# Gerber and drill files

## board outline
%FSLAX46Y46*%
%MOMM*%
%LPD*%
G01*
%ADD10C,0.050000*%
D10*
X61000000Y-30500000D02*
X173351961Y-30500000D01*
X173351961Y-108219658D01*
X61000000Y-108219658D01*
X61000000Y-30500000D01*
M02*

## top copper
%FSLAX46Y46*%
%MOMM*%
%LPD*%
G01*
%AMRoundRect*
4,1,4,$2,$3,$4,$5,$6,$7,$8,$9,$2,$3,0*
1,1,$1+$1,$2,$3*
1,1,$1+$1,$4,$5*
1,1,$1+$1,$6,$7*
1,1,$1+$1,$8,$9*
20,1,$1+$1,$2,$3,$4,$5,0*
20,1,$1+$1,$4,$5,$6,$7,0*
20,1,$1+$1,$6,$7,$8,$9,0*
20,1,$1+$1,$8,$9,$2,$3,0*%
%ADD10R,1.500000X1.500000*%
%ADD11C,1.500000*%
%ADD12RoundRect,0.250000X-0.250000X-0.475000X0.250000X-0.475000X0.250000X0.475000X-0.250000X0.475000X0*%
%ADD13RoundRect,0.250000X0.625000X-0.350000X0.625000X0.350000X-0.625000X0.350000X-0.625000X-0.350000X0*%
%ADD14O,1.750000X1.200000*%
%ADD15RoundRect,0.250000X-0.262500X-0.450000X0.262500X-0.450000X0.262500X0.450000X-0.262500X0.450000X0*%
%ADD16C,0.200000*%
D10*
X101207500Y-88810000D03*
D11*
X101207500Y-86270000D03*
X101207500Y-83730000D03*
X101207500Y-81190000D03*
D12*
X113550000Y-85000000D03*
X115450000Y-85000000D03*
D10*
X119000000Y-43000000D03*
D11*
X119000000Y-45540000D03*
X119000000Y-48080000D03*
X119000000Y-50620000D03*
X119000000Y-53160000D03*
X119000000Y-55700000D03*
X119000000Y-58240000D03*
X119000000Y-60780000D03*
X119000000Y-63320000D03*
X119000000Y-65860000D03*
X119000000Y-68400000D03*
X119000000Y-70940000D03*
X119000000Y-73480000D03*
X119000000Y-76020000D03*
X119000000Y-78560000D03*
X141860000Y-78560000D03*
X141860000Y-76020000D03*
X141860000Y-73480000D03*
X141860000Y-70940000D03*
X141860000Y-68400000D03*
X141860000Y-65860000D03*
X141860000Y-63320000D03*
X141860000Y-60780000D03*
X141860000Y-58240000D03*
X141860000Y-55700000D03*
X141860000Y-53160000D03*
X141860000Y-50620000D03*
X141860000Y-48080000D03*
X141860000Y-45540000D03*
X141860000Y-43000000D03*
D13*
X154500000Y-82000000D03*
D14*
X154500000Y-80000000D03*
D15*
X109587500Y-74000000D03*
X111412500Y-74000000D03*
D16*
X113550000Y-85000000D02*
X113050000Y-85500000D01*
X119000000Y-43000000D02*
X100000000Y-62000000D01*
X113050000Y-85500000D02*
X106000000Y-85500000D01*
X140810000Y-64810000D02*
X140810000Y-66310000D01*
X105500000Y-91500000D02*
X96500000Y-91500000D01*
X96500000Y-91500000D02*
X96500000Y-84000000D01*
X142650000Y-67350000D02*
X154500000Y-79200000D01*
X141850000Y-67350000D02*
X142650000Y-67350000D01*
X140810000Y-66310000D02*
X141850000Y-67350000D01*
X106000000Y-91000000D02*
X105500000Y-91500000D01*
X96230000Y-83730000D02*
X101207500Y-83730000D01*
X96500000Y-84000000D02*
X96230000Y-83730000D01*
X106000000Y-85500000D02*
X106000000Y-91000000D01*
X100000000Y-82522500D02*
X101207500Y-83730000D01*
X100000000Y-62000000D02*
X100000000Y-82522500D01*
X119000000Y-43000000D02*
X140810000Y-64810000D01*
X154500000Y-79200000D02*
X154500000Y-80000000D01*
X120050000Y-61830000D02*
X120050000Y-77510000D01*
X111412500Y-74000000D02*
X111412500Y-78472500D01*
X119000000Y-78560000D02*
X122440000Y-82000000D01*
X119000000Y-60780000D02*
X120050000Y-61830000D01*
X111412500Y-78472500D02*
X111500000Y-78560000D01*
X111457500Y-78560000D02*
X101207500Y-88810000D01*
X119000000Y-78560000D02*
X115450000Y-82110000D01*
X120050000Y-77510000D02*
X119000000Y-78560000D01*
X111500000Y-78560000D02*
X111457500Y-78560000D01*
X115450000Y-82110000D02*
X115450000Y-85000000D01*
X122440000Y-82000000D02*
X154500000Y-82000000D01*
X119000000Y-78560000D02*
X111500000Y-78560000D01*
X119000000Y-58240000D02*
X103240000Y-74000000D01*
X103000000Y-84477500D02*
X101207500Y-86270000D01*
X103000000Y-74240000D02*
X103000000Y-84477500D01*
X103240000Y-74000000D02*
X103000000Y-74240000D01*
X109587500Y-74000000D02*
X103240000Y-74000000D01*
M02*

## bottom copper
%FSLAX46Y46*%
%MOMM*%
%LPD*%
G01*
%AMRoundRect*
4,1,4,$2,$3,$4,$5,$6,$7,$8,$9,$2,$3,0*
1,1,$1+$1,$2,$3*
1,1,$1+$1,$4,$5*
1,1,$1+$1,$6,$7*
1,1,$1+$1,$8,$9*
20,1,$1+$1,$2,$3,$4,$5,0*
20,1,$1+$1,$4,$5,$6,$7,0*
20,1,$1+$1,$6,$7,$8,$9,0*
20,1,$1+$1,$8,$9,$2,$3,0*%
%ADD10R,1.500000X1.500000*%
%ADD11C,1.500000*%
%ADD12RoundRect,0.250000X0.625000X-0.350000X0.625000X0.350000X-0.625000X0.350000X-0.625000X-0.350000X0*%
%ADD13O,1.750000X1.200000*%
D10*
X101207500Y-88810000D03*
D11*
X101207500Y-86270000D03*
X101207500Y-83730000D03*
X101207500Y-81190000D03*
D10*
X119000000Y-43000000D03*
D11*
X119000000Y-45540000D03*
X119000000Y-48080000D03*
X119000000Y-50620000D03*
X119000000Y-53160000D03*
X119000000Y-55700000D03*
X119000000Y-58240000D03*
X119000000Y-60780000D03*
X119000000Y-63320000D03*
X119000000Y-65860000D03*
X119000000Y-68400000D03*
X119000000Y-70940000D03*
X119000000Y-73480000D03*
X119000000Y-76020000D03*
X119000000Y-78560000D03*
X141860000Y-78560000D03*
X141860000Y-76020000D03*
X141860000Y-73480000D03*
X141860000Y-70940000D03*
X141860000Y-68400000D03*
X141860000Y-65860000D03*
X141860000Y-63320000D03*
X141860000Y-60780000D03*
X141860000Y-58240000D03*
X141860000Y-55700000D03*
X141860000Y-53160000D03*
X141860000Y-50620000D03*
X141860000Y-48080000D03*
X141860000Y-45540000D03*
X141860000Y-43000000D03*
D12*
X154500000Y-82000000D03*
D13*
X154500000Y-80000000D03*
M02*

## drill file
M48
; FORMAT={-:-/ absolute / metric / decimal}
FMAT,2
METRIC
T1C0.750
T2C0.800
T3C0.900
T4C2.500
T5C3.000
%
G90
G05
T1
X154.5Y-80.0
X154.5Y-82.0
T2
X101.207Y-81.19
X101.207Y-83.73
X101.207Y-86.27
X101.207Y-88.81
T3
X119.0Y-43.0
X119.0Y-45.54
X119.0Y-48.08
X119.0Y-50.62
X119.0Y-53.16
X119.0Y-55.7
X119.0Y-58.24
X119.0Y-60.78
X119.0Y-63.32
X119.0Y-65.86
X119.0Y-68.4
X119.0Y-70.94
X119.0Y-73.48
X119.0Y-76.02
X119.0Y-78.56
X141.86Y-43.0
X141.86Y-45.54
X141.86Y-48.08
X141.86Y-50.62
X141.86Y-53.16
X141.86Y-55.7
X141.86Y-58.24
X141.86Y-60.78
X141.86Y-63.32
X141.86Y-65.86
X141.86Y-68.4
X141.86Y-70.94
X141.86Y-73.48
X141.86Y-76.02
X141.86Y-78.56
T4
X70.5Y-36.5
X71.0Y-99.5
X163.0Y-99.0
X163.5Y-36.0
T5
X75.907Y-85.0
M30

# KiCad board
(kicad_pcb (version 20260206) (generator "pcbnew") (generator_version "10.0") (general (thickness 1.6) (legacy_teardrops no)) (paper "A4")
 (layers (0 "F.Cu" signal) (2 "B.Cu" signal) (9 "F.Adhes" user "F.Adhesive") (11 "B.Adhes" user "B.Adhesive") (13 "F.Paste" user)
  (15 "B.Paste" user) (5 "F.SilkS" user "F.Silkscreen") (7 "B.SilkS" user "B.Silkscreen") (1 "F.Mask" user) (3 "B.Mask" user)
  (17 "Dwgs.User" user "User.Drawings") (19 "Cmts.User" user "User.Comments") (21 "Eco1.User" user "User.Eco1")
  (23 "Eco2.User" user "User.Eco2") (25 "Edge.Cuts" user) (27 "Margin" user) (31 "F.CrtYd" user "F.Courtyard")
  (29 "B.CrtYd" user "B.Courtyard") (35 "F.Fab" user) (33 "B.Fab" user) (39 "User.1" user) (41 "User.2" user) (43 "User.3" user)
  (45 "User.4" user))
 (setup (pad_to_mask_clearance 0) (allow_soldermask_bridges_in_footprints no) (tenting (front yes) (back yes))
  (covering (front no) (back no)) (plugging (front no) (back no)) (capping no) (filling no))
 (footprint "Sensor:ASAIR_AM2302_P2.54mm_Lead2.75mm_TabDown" (layer "F.Cu") (at 101.2075 88.81 180)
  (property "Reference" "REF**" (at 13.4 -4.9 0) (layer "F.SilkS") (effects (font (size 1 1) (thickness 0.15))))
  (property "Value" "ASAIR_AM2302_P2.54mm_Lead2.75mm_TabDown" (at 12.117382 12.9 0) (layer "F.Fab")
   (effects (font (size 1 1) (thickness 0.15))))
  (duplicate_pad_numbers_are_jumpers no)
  (pad "" np_thru_hole circle (at 25.3 3.81 180) (size 3 3) (drill 3) (layers "*.Cu" "*.Mask"))
  (pad "1" thru_hole rect (at 0 0 180) (size 1.5 1.5) (drill 0.8) (layers "*.Cu" "*.Mask") (remove_unused_layers no) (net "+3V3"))
  (pad "2" thru_hole circle (at 0 2.54 180) (size 1.5 1.5) (drill 0.8) (layers "*.Cu" "*.Mask") (remove_unused_layers no) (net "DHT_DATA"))
  (pad "3" thru_hole circle (at 0 5.08 180) (size 1.5 1.5) (drill 0.8) (layers "*.Cu" "*.Mask") (remove_unused_layers no) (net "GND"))
  (pad "4" thru_hole circle (at 0 7.62 180) (size 1.5 1.5) (drill 0.8) (layers "*.Cu" "*.Mask") (remove_unused_layers no)))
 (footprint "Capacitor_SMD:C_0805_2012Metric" (layer "F.Cu") (at 114.5 85)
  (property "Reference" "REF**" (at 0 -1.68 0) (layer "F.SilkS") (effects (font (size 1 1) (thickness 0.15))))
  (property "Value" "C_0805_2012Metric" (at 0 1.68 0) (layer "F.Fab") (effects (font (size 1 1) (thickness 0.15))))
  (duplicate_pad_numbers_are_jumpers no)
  (pad "1" smd roundrect (at -0.95 0) (size 1 1.45) (layers "F.Cu" "F.Mask" "F.Paste") (roundrect_rratio 0.25) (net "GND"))
  (pad "2" smd roundrect (at 0.95 0) (size 1 1.45) (layers "F.Cu" "F.Mask" "F.Paste") (roundrect_rratio 0.25) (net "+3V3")))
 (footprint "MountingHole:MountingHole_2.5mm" (layer "F.Cu") (at 163 99)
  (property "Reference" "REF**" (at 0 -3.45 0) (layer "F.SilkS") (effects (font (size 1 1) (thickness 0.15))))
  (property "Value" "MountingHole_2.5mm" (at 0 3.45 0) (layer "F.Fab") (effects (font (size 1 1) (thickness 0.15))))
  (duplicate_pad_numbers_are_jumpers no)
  (pad "" np_thru_hole circle (at 0 0) (size 2.5 2.5) (drill 2.5) (layers "*.Cu" "*.Mask")))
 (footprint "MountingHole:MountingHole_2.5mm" (layer "F.Cu") (at 71 99.5)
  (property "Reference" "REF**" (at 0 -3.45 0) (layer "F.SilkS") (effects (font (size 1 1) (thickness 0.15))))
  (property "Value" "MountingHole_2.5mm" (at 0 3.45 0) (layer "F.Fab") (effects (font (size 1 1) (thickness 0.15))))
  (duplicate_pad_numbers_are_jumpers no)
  (pad "" np_thru_hole circle (at 0 0) (size 2.5 2.5) (drill 2.5) (layers "*.Cu" "*.Mask")))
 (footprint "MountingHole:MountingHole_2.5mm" (layer "F.Cu") (at 163.5 36)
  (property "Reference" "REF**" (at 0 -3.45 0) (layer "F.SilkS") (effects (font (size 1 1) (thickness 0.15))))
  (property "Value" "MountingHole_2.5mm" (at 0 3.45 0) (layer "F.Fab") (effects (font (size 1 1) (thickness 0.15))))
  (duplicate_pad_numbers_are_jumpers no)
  (pad "" np_thru_hole circle (at 0 0) (size 2.5 2.5) (drill 2.5) (layers "*.Cu" "*.Mask")))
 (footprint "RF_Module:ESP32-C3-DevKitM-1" (layer "F.Cu") (at 119 43)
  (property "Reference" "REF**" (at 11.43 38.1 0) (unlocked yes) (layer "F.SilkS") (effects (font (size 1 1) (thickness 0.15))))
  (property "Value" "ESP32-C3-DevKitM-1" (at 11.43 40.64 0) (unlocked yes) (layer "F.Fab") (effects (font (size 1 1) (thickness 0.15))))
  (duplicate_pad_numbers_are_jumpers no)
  (pad "1" thru_hole rect (at 0 0) (size 1.5 1.5) (drill 0.9) (layers "*.Cu" "*.Mask") (remove_unused_layers yes) (keep_end_layers yes)
   (zone_layer_connections) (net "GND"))
  (pad "2" thru_hole circle (at 0 2.54) (size 1.5 1.5) (drill 0.9) (layers "*.Cu" "*.Mask") (remove_unused_layers yes) (keep_end_layers yes)
   (zone_layer_connections))
  (pad "3" thru_hole circle (at 0 5.08) (size 1.5 1.5) (drill 0.9) (layers "*.Cu" "*.Mask") (remove_unused_layers yes) (keep_end_layers yes)
   (zone_layer_connections))
  (pad "4" thru_hole circle (at 0 7.62) (size 1.5 1.5) (drill 0.9) (layers "*.Cu" "*.Mask") (remove_unused_layers yes) (keep_end_layers yes)
   (zone_layer_connections))
  (pad "5" thru_hole circle (at 0 10.16) (size 1.5 1.5) (drill 0.9) (layers "*.Cu" "*.Mask") (remove_unused_layers yes)
   (keep_end_layers yes) (zone_layer_connections))
  (pad "6" thru_hole circle (at 0 12.7) (size 1.5 1.5) (drill 0.9) (layers "*.Cu" "*.Mask") (remove_unused_layers yes) (keep_end_layers yes)
   (zone_layer_connections))
  (pad "7" thru_hole circle (at 0 15.24) (size 1.5 1.5) (drill 0.9) (layers "*.Cu" "*.Mask") (remove_unused_layers yes)
   (keep_end_layers yes) (zone_layer_connections) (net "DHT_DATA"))
  (pad "8" thru_hole circle (at 0 17.78) (size 1.5 1.5) (drill 0.9) (layers "*.Cu" "*.Mask") (remove_unused_layers yes)
   (keep_end_layers yes) (zone_layer_connections) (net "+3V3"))
  (pad "9" thru_hole circle (at 0 20.32) (size 1.5 1.5) (drill 0.9) (layers "*.Cu" "*.Mask") (remove_unused_layers yes)
   (keep_end_layers yes) (zone_layer_connections))
  (pad "10" thru_hole circle (at 0 22.86) (size 1.5 1.5) (drill 0.9) (layers "*.Cu" "*.Mask") (remove_unused_layers yes)
   (keep_end_layers yes) (zone_layer_connections))
  (pad "11" thru_hole circle (at 0 25.4) (size 1.5 1.5) (drill 0.9) (layers "*.Cu" "*.Mask") (remove_unused_layers yes)
   (keep_end_layers yes) (zone_layer_connections))
  (pad "12" thru_hole circle (at 0 27.94) (size 1.5 1.5) (drill 0.9) (layers "*.Cu" "*.Mask") (remove_unused_layers yes)
   (keep_end_layers yes) (zone_layer_connections))
  (pad "13" thru_hole circle (at 0 30.48) (size 1.5 1.5) (drill 0.9) (layers "*.Cu" "*.Mask") (remove_unused_layers yes)
   (keep_end_layers yes) (zone_layer_connections))
  (pad "14" thru_hole circle (at 0 33.02) (size 1.5 1.5) (drill 0.9) (layers "*.Cu" "*.Mask") (remove_unused_layers yes)
   (keep_end_layers yes) (zone_layer_connections))
  (pad "15" thru_hole circle (at 0 35.56) (size 1.5 1.5) (drill 0.9) (layers "*.Cu" "*.Mask") (remove_unused_layers yes)
   (keep_end_layers yes) (zone_layer_connections) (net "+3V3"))
  (pad "16" thru_hole circle (at 22.86 35.56) (size 1.5 1.5) (drill 0.9) (layers "*.Cu" "*.Mask") (remove_unused_layers yes)
   (keep_end_layers yes) (zone_layer_connections))
  (pad "17" thru_hole circle (at 22.86 33.02) (size 1.5 1.5) (drill 0.9) (layers "*.Cu" "*.Mask") (remove_unused_layers yes)
   (keep_end_layers yes) (zone_layer_connections))
  (pad "18" thru_hole circle (at 22.86 30.48) (size 1.5 1.5) (drill 0.9) (layers "*.Cu" "*.Mask") (remove_unused_layers yes)
   (keep_end_layers yes) (zone_layer_connections))
  (pad "19" thru_hole circle (at 22.86 27.94) (size 1.5 1.5) (drill 0.9) (layers "*.Cu" "*.Mask") (remove_unused_layers yes)
   (keep_end_layers yes) (zone_layer_connections))
  (pad "20" thru_hole circle (at 22.86 25.4) (size 1.5 1.5) (drill 0.9) (layers "*.Cu" "*.Mask") (remove_unused_layers yes)
   (keep_end_layers yes) (zone_layer_connections))
  (pad "21" thru_hole circle (at 22.86 22.86) (size 1.5 1.5) (drill 0.9) (layers "*.Cu" "*.Mask") (remove_unused_layers yes)
   (keep_end_layers yes) (zone_layer_connections))
  (pad "22" thru_hole circle (at 22.86 20.32) (size 1.5 1.5) (drill 0.9) (layers "*.Cu" "*.Mask") (remove_unused_layers yes)
   (keep_end_layers yes) (zone_layer_connections))
  (pad "23" thru_hole circle (at 22.86 17.78) (size 1.5 1.5) (drill 0.9) (layers "*.Cu" "*.Mask") (remove_unused_layers yes)
   (keep_end_layers yes) (zone_layer_connections))
  (pad "24" thru_hole circle (at 22.86 15.24) (size 1.5 1.5) (drill 0.9) (layers "*.Cu" "*.Mask") (remove_unused_layers yes)
   (keep_end_layers yes) (zone_layer_connections))
  (pad "25" thru_hole circle (at 22.86 12.7) (size 1.5 1.5) (drill 0.9) (layers "*.Cu" "*.Mask") (remove_unused_layers yes)
   (keep_end_layers yes) (zone_layer_connections))
  (pad "26" thru_hole circle (at 22.86 10.16) (size 1.5 1.5) (drill 0.9) (layers "*.Cu" "*.Mask") (remove_unused_layers yes)
   (keep_end_layers yes) (zone_layer_connections))
  (pad "27" thru_hole circle (at 22.86 7.62) (size 1.5 1.5) (drill 0.9) (layers "*.Cu" "*.Mask") (remove_unused_layers yes)
   (keep_end_layers yes) (zone_layer_connections))
  (pad "28" thru_hole circle (at 22.86 5.08) (size 1.5 1.5) (drill 0.9) (layers "*.Cu" "*.Mask") (remove_unused_layers yes)
   (keep_end_layers yes) (zone_layer_connections))
  (pad "29" thru_hole circle (at 22.86 2.54) (size 1.5 1.5) (drill 0.9) (layers "*.Cu" "*.Mask") (remove_unused_layers yes)
   (keep_end_layers yes) (zone_layer_connections))
  (pad "30" thru_hole circle (at 22.86 0) (size 1.5 1.5) (drill 0.9) (layers "*.Cu" "*.Mask") (remove_unused_layers yes)
   (keep_end_layers yes) (zone_layer_connections)))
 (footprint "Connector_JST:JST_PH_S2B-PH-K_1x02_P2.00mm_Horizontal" (layer "F.Cu") (at 154.5 82 90)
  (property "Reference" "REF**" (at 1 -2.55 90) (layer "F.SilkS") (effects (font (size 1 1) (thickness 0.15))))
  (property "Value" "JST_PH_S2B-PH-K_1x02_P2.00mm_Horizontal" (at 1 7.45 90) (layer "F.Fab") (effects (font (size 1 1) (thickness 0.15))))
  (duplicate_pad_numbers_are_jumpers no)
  (pad "1" thru_hole roundrect (at 0 0 90) (size 1.2 1.75) (drill 0.75) (layers "*.Cu" "*.Mask") (remove_unused_layers no)
   (roundrect_rratio 0.208333) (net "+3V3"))
  (pad "2" thru_hole oval (at 2 0 90) (size 1.2 1.75) (drill 0.75) (layers "*.Cu" "*.Mask") (remove_unused_layers no) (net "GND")))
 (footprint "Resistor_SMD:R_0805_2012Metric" (layer "F.Cu") (at 110.5 74)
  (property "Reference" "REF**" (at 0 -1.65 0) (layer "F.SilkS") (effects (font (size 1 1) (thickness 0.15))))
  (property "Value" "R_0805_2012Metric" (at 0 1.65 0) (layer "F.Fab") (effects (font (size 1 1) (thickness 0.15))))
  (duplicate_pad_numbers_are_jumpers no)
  (pad "1" smd roundrect (at -0.9125 0) (size 1.025 1.4) (layers "F.Cu" "F.Mask" "F.Paste") (roundrect_rratio 0.243902) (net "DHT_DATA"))
  (pad "2" smd roundrect (at 0.9125 0) (size 1.025 1.4) (layers "F.Cu" "F.Mask" "F.Paste") (roundrect_rratio 0.243902) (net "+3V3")))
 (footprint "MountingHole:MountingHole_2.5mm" (layer "F.Cu") (at 70.5 36.5)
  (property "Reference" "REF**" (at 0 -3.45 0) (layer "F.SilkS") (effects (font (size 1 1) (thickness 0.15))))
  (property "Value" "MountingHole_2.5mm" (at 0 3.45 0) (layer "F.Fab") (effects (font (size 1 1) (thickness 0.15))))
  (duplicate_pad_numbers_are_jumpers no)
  (pad "" np_thru_hole circle (at 0 0) (size 2.5 2.5) (drill 2.5) (layers "*.Cu" "*.Mask")))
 (gr_rect (start 61 30.5) (end 173.351961 108.219658) (stroke (width 0.05) (type default)) (fill no) (layer "Edge.Cuts"))
 (segment (start 113.55 85) (end 113.05 85.5) (width 0.2) (layer "F.Cu") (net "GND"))
 (segment (start 119 43) (end 100 62) (width 0.2) (layer "F.Cu") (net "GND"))
 (segment (start 113.05 85.5) (end 106 85.5) (width 0.2) (layer "F.Cu") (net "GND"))
 (segment (start 140.81 64.81) (end 140.81 66.31) (width 0.2) (layer "F.Cu") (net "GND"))
 (segment (start 105.5 91.5) (end 96.5 91.5) (width 0.2) (layer "F.Cu") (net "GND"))
 (segment (start 96.5 91.5) (end 96.5 84) (width 0.2) (layer "F.Cu") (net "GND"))
 (segment (start 142.65 67.35) (end 154.5 79.2) (width 0.2) (layer "F.Cu") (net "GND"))
 (segment (start 141.85 67.35) (end 142.65 67.35) (width 0.2) (layer "F.Cu") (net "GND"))
 (segment (start 140.81 66.31) (end 141.85 67.35) (width 0.2) (layer "F.Cu") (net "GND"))
 (segment (start 106 91) (end 105.5 91.5) (width 0.2) (layer "F.Cu") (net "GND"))
 (segment (start 96.23 83.73) (end 101.2075 83.73) (width 0.2) (layer "F.Cu") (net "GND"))
 (segment (start 96.5 84) (end 96.23 83.73) (width 0.2) (layer "F.Cu") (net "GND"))
 (segment (start 106 85.5) (end 106 91) (width 0.2) (layer "F.Cu") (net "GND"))
 (segment (start 100 82.5225) (end 101.2075 83.73) (width 0.2) (layer "F.Cu") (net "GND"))
 (segment (start 100 62) (end 100 82.5225) (width 0.2) (layer "F.Cu") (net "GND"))
 (segment (start 119 43) (end 140.81 64.81) (width 0.2) (layer "F.Cu") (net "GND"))
 (segment (start 154.5 79.2) (end 154.5 80) (width 0.2) (layer "F.Cu") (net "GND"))
 (segment (start 120.05 61.83) (end 120.05 77.51) (width 0.2) (layer "F.Cu") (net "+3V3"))
 (segment (start 111.4125 74) (end 111.4125 78.4725) (width 0.2) (layer "F.Cu") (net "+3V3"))
 (segment (start 119 78.56) (end 122.44 82) (width 0.2) (layer "F.Cu") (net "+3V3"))
 (segment (start 119 60.78) (end 120.05 61.83) (width 0.2) (layer "F.Cu") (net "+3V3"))
 (segment (start 111.4125 78.4725) (end 111.5 78.56) (width 0.2) (layer "F.Cu") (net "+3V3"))
 (segment (start 111.4575 78.56) (end 101.2075 88.81) (width 0.2) (layer "F.Cu") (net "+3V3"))
 (segment (start 119 78.56) (end 115.45 82.11) (width 0.2) (layer "F.Cu") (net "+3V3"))
 (segment (start 120.05 77.51) (end 119 78.56) (width 0.2) (layer "F.Cu") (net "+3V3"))
 (segment (start 111.5 78.56) (end 111.4575 78.56) (width 0.2) (layer "F.Cu") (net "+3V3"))
 (segment (start 115.45 82.11) (end 115.45 85) (width 0.2) (layer "F.Cu") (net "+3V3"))
 (segment (start 122.44 82) (end 154.5 82) (width 0.2) (layer "F.Cu") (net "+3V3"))
 (segment (start 119 78.56) (end 111.5 78.56) (width 0.2) (layer "F.Cu") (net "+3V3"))
 (segment (start 119 58.24) (end 103.24 74) (width 0.2) (layer "F.Cu") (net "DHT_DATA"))
 (segment (start 103 84.4775) (end 101.2075 86.27) (width 0.2) (layer "F.Cu") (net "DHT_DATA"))
 (segment (start 103 74.24) (end 103 84.4775) (width 0.2) (layer "F.Cu") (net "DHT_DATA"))
 (segment (start 103.24 74) (end 103 74.24) (width 0.2) (layer "F.Cu") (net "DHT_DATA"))
 (segment (start 109.5875 74) (end 103.24 74) (width 0.2) (layer "F.Cu") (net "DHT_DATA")))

